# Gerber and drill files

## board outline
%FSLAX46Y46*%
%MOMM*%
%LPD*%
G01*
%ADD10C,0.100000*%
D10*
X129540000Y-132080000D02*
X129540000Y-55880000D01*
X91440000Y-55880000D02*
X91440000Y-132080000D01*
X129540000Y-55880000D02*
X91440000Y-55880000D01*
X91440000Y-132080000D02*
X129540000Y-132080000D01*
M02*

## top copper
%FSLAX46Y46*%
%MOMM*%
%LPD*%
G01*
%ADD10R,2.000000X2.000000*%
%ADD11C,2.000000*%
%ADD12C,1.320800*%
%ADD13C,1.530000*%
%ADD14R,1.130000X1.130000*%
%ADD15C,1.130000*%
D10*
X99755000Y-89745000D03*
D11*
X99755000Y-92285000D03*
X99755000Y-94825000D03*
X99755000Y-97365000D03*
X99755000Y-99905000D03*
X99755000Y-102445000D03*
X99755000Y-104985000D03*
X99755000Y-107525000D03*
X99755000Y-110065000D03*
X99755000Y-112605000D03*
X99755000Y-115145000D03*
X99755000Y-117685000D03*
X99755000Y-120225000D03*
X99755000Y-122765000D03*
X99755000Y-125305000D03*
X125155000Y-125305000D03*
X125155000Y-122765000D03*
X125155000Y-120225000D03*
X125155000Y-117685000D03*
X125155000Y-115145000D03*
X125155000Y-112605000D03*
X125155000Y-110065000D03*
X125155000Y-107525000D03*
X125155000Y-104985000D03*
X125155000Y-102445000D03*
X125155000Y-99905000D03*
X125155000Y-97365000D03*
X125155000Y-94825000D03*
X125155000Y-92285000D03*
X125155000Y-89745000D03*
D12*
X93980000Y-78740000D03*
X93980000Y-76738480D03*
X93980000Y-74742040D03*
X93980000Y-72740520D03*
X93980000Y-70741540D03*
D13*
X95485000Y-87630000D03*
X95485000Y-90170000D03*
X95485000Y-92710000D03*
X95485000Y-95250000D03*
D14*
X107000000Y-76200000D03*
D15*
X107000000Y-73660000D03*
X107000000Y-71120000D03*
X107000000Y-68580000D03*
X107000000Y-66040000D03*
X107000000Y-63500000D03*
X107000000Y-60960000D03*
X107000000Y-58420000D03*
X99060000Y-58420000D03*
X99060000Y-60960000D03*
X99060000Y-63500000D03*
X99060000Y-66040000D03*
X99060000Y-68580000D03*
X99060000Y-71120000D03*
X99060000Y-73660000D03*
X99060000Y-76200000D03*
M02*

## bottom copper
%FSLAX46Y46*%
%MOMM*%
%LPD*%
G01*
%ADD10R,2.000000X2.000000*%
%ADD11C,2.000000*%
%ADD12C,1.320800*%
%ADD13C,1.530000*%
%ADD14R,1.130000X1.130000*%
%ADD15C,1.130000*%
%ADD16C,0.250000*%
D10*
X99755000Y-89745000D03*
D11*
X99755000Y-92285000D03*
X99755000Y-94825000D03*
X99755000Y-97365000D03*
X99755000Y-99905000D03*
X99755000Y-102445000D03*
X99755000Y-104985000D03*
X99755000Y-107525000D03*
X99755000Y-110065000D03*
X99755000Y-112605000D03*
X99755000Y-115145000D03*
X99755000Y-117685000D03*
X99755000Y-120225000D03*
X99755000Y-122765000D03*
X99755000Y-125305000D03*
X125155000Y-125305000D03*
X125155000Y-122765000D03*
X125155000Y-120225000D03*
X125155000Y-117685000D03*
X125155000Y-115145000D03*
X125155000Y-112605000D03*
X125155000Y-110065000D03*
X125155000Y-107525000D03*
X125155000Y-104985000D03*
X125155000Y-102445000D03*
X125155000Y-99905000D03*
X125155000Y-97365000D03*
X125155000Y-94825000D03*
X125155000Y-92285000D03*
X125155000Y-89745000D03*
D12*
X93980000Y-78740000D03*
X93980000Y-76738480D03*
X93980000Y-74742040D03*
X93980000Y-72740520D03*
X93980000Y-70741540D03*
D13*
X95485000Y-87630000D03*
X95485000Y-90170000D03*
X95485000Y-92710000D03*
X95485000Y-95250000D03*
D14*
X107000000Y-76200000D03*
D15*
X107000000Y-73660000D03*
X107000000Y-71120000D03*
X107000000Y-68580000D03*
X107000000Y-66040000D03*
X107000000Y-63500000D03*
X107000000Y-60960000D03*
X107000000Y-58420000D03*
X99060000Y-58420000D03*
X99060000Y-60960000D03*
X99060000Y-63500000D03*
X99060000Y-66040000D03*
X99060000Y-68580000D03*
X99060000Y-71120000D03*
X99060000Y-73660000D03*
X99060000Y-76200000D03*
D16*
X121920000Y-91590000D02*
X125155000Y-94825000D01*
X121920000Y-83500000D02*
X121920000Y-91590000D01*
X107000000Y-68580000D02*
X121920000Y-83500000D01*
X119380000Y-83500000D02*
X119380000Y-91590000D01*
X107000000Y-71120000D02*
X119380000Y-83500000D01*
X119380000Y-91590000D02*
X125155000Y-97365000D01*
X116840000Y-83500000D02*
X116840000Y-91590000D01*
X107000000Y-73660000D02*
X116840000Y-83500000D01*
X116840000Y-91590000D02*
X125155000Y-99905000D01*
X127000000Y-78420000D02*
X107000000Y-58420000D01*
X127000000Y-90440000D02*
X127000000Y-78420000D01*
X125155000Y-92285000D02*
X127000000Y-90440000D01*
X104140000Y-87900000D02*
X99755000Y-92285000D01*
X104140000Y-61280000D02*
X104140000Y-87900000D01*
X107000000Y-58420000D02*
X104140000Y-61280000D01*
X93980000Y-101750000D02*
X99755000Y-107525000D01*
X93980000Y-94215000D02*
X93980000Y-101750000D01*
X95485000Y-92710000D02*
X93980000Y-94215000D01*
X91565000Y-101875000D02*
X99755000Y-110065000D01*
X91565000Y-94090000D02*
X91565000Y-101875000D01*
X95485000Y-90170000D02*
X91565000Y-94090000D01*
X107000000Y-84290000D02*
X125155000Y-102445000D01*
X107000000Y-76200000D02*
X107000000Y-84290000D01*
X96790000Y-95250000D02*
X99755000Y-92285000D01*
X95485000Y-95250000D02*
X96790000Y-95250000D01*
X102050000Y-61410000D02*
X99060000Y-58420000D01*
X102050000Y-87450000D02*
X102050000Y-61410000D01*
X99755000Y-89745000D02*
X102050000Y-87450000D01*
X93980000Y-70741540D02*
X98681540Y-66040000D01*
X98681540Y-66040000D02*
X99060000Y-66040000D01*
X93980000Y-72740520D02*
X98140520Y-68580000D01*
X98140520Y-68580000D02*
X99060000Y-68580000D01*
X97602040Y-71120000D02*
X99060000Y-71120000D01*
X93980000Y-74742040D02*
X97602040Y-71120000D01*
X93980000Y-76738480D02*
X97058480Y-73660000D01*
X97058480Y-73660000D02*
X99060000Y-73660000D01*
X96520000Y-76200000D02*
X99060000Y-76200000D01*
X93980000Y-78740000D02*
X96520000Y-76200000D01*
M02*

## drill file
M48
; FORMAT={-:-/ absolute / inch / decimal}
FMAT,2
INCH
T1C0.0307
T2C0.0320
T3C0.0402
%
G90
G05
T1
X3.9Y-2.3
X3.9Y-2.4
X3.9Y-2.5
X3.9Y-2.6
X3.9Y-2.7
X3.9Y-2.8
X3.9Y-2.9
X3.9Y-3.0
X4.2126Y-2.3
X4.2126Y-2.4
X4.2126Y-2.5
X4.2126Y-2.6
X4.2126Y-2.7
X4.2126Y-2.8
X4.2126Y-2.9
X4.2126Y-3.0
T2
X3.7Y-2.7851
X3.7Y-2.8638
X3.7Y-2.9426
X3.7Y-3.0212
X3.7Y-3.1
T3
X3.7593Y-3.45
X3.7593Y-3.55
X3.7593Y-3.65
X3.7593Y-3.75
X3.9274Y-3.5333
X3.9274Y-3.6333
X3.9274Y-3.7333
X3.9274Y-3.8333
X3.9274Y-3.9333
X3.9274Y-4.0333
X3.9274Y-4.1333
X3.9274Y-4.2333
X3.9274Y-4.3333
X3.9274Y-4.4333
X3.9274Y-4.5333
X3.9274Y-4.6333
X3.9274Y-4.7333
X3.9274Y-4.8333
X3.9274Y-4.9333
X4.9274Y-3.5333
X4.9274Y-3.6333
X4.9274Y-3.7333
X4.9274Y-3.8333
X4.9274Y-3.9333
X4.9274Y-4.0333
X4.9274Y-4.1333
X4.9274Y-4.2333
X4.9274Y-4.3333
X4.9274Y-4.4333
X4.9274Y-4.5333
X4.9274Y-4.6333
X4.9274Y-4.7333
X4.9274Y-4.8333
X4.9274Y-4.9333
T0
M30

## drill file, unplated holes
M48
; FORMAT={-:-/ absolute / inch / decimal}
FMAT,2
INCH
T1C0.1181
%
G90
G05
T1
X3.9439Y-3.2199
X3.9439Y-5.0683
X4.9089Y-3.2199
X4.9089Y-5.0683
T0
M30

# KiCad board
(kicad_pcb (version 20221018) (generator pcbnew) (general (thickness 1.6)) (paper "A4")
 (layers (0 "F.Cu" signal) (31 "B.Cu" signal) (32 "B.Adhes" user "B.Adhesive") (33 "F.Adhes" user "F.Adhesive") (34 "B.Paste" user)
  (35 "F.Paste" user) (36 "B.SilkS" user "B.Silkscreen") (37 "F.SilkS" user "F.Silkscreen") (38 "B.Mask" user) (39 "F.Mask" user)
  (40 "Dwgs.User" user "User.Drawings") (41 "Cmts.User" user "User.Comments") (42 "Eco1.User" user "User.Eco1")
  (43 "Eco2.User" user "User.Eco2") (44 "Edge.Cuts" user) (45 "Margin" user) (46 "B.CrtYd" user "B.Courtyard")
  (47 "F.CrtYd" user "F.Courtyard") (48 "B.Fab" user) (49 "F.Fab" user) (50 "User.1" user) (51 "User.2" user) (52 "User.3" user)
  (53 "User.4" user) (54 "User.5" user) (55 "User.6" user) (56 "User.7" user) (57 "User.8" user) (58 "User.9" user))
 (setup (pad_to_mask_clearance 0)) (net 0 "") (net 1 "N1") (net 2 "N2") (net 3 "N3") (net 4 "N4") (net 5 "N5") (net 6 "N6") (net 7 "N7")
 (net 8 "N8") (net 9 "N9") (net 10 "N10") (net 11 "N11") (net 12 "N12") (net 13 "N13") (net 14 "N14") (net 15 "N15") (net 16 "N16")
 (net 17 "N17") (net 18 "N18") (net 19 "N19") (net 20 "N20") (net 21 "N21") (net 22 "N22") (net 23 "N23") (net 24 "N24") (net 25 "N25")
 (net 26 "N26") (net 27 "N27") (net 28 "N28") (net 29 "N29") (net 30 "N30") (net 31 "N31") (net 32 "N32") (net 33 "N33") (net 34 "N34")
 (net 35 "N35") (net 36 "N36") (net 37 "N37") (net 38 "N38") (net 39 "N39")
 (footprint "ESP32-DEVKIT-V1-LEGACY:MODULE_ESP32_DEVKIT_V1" (layer "F.Cu") (at 112.455 105.26)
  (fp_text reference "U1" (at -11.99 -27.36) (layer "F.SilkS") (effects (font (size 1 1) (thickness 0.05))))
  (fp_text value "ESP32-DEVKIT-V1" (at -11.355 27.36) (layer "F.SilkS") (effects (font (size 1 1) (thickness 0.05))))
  (pad "" np_thru_hole circle (at -12.28 -23.475) (size 3 3) (drill 3) (layers "*.Cu" "*.Mask"))
  (pad "" np_thru_hole circle (at -12.28 23.475) (size 3 3) (drill 3) (layers "*.Cu" "*.Mask"))
  (pad "" np_thru_hole circle (at 12.23 -23.475) (size 3 3) (drill 3) (layers "*.Cu" "*.Mask"))
  (pad "" np_thru_hole circle (at 12.23 23.475) (size 3 3) (drill 3) (layers "*.Cu" "*.Mask"))
  (pad "1" thru_hole rect (at -12.7 -15.515) (size 2 2) (drill 1.02) (layers "*.Cu" "*.Mask") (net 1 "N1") (thermal_bridge_angle 45))
  (pad "2" thru_hole circle (at -12.7 -12.975) (size 2 2) (drill 1.02) (layers "*.Cu" "*.Mask") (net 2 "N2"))
  (pad "3" thru_hole circle (at -12.7 -10.435) (size 2 2) (drill 1.02) (layers "*.Cu" "*.Mask") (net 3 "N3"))
  (pad "4" thru_hole circle (at -12.7 -7.895) (size 2 2) (drill 1.02) (layers "*.Cu" "*.Mask") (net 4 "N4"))
  (pad "5" thru_hole circle (at -12.7 -5.355) (size 2 2) (drill 1.02) (layers "*.Cu" "*.Mask") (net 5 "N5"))
  (pad "6" thru_hole circle (at -12.7 -2.815) (size 2 2) (drill 1.02) (layers "*.Cu" "*.Mask") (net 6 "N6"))
  (pad "7" thru_hole circle (at -12.7 -0.275) (size 2 2) (drill 1.02) (layers "*.Cu" "*.Mask") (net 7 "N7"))
  (pad "8" thru_hole circle (at -12.7 2.265) (size 2 2) (drill 1.02) (layers "*.Cu" "*.Mask") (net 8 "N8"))
  (pad "9" thru_hole circle (at -12.7 4.805) (size 2 2) (drill 1.02) (layers "*.Cu" "*.Mask") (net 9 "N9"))
  (pad "10" thru_hole circle (at -12.7 7.345) (size 2 2) (drill 1.02) (layers "*.Cu" "*.Mask") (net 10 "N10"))
  (pad "11" thru_hole circle (at -12.7 9.885) (size 2 2) (drill 1.02) (layers "*.Cu" "*.Mask") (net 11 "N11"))
  (pad "12" thru_hole circle (at -12.7 12.425) (size 2 2) (drill 1.02) (layers "*.Cu" "*.Mask") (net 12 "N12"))
  (pad "13" thru_hole circle (at -12.7 14.965) (size 2 2) (drill 1.02) (layers "*.Cu" "*.Mask") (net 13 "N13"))
  (pad "14" thru_hole circle (at -12.7 17.505) (size 2 2) (drill 1.02) (layers "*.Cu" "*.Mask") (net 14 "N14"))
  (pad "15" thru_hole circle (at -12.7 20.045) (size 2 2) (drill 1.02) (layers "*.Cu" "*.Mask") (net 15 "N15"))
  (pad "16" thru_hole circle (at 12.7 20.045) (size 2 2) (drill 1.02) (layers "*.Cu" "*.Mask") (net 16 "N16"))
  (pad "17" thru_hole circle (at 12.7 17.505) (size 2 2) (drill 1.02) (layers "*.Cu" "*.Mask") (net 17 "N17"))
  (pad "18" thru_hole circle (at 12.7 14.965) (size 2 2) (drill 1.02) (layers "*.Cu" "*.Mask") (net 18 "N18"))
  (pad "19" thru_hole circle (at 12.7 12.425) (size 2 2) (drill 1.02) (layers "*.Cu" "*.Mask") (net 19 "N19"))
  (pad "20" thru_hole circle (at 12.7 9.885) (size 2 2) (drill 1.02) (layers "*.Cu" "*.Mask") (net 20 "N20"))
  (pad "21" thru_hole circle (at 12.7 7.345) (size 2 2) (drill 1.02) (layers "*.Cu" "*.Mask") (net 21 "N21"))
  (pad "22" thru_hole circle (at 12.7 4.805) (size 2 2) (drill 1.02) (layers "*.Cu" "*.Mask") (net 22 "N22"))
  (pad "23" thru_hole circle (at 12.7 2.265) (size 2 2) (drill 1.02) (layers "*.Cu" "*.Mask") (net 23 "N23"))
  (pad "24" thru_hole circle (at 12.7 -0.275) (size 2 2) (drill 1.02) (layers "*.Cu" "*.Mask") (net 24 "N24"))
  (pad "25" thru_hole circle (at 12.7 -2.815) (size 2 2) (drill 1.02) (layers "*.Cu" "*.Mask") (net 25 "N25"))
  (pad "26" thru_hole circle (at 12.7 -5.355) (size 2 2) (drill 1.02) (layers "*.Cu" "*.Mask") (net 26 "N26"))
  (pad "27" thru_hole circle (at 12.7 -7.895) (size 2 2) (drill 1.02) (layers "*.Cu" "*.Mask") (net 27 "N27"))
  (pad "28" thru_hole circle (at 12.7 -10.435) (size 2 2) (drill 1.02) (layers "*.Cu" "*.Mask") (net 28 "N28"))
  (pad "29" thru_hole circle (at 12.7 -12.975) (size 2 2) (drill 1.02) (layers "*.Cu" "*.Mask") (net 2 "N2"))
  (pad "30" thru_hole circle (at 12.7 -15.515) (size 2 2) (drill 1.02) (layers "*.Cu" "*.Mask") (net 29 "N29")))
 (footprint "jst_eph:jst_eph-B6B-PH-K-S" (layer "F.Cu") (at 93.98 75.74026 -90)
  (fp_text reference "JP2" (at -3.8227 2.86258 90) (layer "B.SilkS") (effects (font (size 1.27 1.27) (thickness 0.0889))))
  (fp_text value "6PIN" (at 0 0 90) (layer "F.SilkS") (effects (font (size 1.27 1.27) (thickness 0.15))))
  (pad "2" thru_hole circle (at 2.99974 0 270) (size 1.3208 1.3208) (drill 0.8128) (layers "F&B.Cu" "F.Paste" "F.SilkS" "F.Mask")
   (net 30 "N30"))
  (pad "3" thru_hole circle (at 0.99822 0 270) (size 1.3208 1.3208) (drill 0.8128) (layers "F&B.Cu" "F.Paste" "F.SilkS" "F.Mask")
   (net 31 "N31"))
  (pad "4" thru_hole circle (at -0.99822 0 270) (size 1.3208 1.3208) (drill 0.8128) (layers "F&B.Cu" "F.Paste" "F.SilkS" "F.Mask")
   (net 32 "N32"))
  (pad "5" thru_hole circle (at -2.99974 0 270) (size 1.3208 1.3208) (drill 0.8128) (layers "F&B.Cu" "F.Paste" "F.SilkS" "F.Mask")
   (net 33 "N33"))
  (pad "6" thru_hole circle (at -4.99872 0 270) (size 1.3208 1.3208) (drill 0.8128) (layers "F&B.Cu" "F.Paste" "F.SilkS" "F.Mask")
   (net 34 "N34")))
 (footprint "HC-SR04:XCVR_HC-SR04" (layer "F.Cu") (at 95.485 91.44 -90)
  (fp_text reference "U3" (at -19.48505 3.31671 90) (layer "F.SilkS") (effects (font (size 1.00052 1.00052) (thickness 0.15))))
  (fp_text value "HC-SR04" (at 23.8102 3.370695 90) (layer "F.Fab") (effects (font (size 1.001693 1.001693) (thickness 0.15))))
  (pad "1" thru_hole circle (at -3.81 0 270) (size 1.53 1.53) (drill 1.02) (layers "*.Cu" "*.Mask") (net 1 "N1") (solder_mask_margin 0.102))
  (pad "2" thru_hole circle (at -1.27 0 270) (size 1.53 1.53) (drill 1.02) (layers "*.Cu" "*.Mask") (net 9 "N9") (solder_mask_margin 0.102))
  (pad "3" thru_hole circle (at 1.27 0 270) (size 1.53 1.53) (drill 1.02) (layers "*.Cu" "*.Mask") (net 8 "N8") (solder_mask_margin 0.102))
  (pad "4" thru_hole circle (at 3.81 0 270) (size 1.53 1.53) (drill 1.02) (layers "*.Cu" "*.Mask") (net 2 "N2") (solder_mask_margin 0.102)))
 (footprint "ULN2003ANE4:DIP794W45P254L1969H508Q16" (layer "F.Cu") (at 103.03 67.31 180)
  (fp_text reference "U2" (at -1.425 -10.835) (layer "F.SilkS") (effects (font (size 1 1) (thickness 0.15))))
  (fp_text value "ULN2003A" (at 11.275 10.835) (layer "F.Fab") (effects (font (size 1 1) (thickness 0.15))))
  (pad "1" thru_hole rect (at -3.97 -8.89 180) (size 1.13 1.13) (drill 0.78) (layers "*.Cu" "*.Mask") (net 25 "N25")
   (solder_mask_margin 0.102))
  (pad "2" thru_hole circle (at -3.97 -6.35 180) (size 1.13 1.13) (drill 0.78) (layers "*.Cu" "*.Mask") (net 26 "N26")
   (solder_mask_margin 0.102))
  (pad "3" thru_hole circle (at -3.97 -3.81 180) (size 1.13 1.13) (drill 0.78) (layers "*.Cu" "*.Mask") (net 27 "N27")
   (solder_mask_margin 0.102))
  (pad "4" thru_hole circle (at -3.97 -1.27 180) (size 1.13 1.13) (drill 0.78) (layers "*.Cu" "*.Mask") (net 28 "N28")
   (solder_mask_margin 0.102))
  (pad "5" thru_hole circle (at -3.97 1.27 180) (size 1.13 1.13) (drill 0.78) (layers "*.Cu" "*.Mask") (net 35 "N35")
   (solder_mask_margin 0.102))
  (pad "6" thru_hole circle (at -3.97 3.81 180) (size 1.13 1.13) (drill 0.78) (layers "*.Cu" "*.Mask") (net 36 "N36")
   (solder_mask_margin 0.102))
  (pad "7" thru_hole circle (at -3.97 6.35 180) (size 1.13 1.13) (drill 0.78) (layers "*.Cu" "*.Mask") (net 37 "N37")
   (solder_mask_margin 0.102))
  (pad "8" thru_hole circle (at -3.97 8.89 180) (size 1.13 1.13) (drill 0.78) (layers "*.Cu" "*.Mask") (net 2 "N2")
   (solder_mask_margin 0.102))
  (pad "9" thru_hole circle (at 3.97 8.89 180) (size 1.13 1.13) (drill 0.78) (layers "*.Cu" "*.Mask") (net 1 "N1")
   (solder_mask_margin 0.102))
  (pad "10" thru_hole circle (at 3.97 6.35 180) (size 1.13 1.13) (drill 0.78) (layers "*.Cu" "*.Mask") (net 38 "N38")
   (solder_mask_margin 0.102))
  (pad "11" thru_hole circle (at 3.97 3.81 180) (size 1.13 1.13) (drill 0.78) (layers "*.Cu" "*.Mask") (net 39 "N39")
   (solder_mask_margin 0.102))
  (pad "12" thru_hole circle (at 3.97 1.27 180) (size 1.13 1.13) (drill 0.78) (layers "*.Cu" "*.Mask") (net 34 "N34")
   (solder_mask_margin 0.102))
  (pad "13" thru_hole circle (at 3.97 -1.27 180) (size 1.13 1.13) (drill 0.78) (layers "*.Cu" "*.Mask") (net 33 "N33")
   (solder_mask_margin 0.102))
  (pad "14" thru_hole circle (at 3.97 -3.81 180) (size 1.13 1.13) (drill 0.78) (layers "*.Cu" "*.Mask") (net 32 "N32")
   (solder_mask_margin 0.102))
  (pad "15" thru_hole circle (at 3.97 -6.35 180) (size 1.13 1.13) (drill 0.78) (layers "*.Cu" "*.Mask") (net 31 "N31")
   (solder_mask_margin 0.102))
  (pad "16" thru_hole circle (at 3.97 -8.89 180) (size 1.13 1.13) (drill 0.78) (layers "*.Cu" "*.Mask") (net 30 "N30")
   (solder_mask_margin 0.102)))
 (gr_line (start 129.54 132.08) (end 129.54 55.88) (stroke (width 0.1) (type default)) (layer "Edge.Cuts"))
 (gr_line (start 91.44 55.88) (end 91.44 132.08) (stroke (width 0.1) (type default)) (layer "Edge.Cuts"))
 (gr_line (start 129.54 55.88) (end 91.44 55.88) (stroke (width 0.1) (type default)) (layer "Edge.Cuts"))
 (gr_line (start 91.44 132.08) (end 129.54 132.08) (stroke (width 0.1) (type default)) (layer "Edge.Cuts"))
 (segment (start 107 84.29) (end 125.155 102.445) (width 0.25) (layer "B.Cu") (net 25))
 (segment (start 107 76.2) (end 107 84.29) (width 0.25) (layer "B.Cu") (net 25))
 (segment (start 116.84 83.5) (end 116.84 91.59) (width 0.25) (layer "B.Cu") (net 26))
 (segment (start 116.84 91.59) (end 125.155 99.905) (width 0.25) (layer "B.Cu") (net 26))
 (segment (start 107 73.66) (end 116.84 83.5) (width 0.25) (layer "B.Cu") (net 26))
 (segment (start 107 71.12) (end 119.38 83.5) (width 0.25) (layer "B.Cu") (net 27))
 (segment (start 119.38 83.5) (end 119.38 91.59) (width 0.25) (layer "B.Cu") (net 27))
 (segment (start 119.38 91.59) (end 125.155 97.365) (width 0.25) (layer "B.Cu") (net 27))
 (segment (start 121.92 91.59) (end 125.155 94.825) (width 0.25) (layer "B.Cu") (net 28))
 (segment (start 121.92 83.5) (end 121.92 91.59) (width 0.25) (layer "B.Cu") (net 28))
 (segment (start 107 68.58) (end 121.92 83.5) (width 0.25) (layer "B.Cu") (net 28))
 (segment (start 96.79 95.25) (end 99.755 92.285) (width 0.25) (layer "B.Cu") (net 2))
 (segment (start 127 90.44) (end 127 78.42) (width 0.25) (layer "B.Cu") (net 2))
 (segment (start 125.155 92.285) (end 127 90.44) (width 0.25) (layer "B.Cu") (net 2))
 (segment (start 95.485 95.25) (end 96.79 95.25) (width 0.25) (layer "B.Cu") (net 2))
 (segment (start 107 58.42) (end 104.14 61.28) (width 0.25) (layer "B.Cu") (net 2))
 (segment (start 104.14 61.28) (end 104.14 87.9) (width 0.25) (layer "B.Cu") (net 2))
 (segment (start 127 78.42) (end 107 58.42) (width 0.25) (layer "B.Cu") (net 2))
 (segment (start 104.14 87.9) (end 99.755 92.285) (width 0.25) (layer "B.Cu") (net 2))
 (segment (start 102.05 61.41) (end 99.06 58.42) (width 0.25) (layer "B.Cu") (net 1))
 (segment (start 102.05 87.45) (end 102.05 61.41) (width 0.25) (layer "B.Cu") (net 1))
 (segment (start 99.755 89.745) (end 102.05 87.45) (width 0.25) (layer "B.Cu") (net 1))
 (segment (start 93.98 101.75) (end 99.755 107.525) (width 0.25) (layer "B.Cu") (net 8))
 (segment (start 93.98 94.215) (end 93.98 101.75) (width 0.25) (layer "B.Cu") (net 8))
 (segment (start 95.485 92.71) (end 93.98 94.215) (width 0.25) (layer "B.Cu") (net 8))
 (segment (start 91.565 94.09) (end 91.565 101.875) (width 0.25) (layer "B.Cu") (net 9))
 (segment (start 95.485 90.17) (end 91.565 94.09) (width 0.25) (layer "B.Cu") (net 9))
 (segment (start 91.565 101.875) (end 99.755 110.065) (width 0.25) (layer "B.Cu") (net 9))
 (segment (start 93.98 70.74154) (end 98.68154 66.04) (width 0.25) (layer "B.Cu") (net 34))
 (segment (start 98.68154 66.04) (end 99.06 66.04) (width 0.25) (layer "B.Cu") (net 34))
 (segment (start 93.98 72.74052) (end 98.14052 68.58) (width 0.25) (layer "B.Cu") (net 33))
 (segment (start 98.14052 68.58) (end 99.06 68.58) (width 0.25) (layer "B.Cu") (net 33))
 (segment (start 97.60204 71.12) (end 99.06 71.12) (width 0.25) (layer "B.Cu") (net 32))
 (segment (start 93.98 74.74204) (end 97.60204 71.12) (width 0.25) (layer "B.Cu") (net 32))
 (segment (start 93.98 76.73848) (end 97.05848 73.66) (width 0.25) (layer "B.Cu") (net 31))
 (segment (start 97.05848 73.66) (end 99.06 73.66) (width 0.25) (layer "B.Cu") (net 31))
 (segment (start 96.52 76.2) (end 99.06 76.2) (width 0.25) (layer "B.Cu") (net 30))
 (segment (start 93.98 78.74) (end 96.52 76.2) (width 0.25) (layer "B.Cu") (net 30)))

